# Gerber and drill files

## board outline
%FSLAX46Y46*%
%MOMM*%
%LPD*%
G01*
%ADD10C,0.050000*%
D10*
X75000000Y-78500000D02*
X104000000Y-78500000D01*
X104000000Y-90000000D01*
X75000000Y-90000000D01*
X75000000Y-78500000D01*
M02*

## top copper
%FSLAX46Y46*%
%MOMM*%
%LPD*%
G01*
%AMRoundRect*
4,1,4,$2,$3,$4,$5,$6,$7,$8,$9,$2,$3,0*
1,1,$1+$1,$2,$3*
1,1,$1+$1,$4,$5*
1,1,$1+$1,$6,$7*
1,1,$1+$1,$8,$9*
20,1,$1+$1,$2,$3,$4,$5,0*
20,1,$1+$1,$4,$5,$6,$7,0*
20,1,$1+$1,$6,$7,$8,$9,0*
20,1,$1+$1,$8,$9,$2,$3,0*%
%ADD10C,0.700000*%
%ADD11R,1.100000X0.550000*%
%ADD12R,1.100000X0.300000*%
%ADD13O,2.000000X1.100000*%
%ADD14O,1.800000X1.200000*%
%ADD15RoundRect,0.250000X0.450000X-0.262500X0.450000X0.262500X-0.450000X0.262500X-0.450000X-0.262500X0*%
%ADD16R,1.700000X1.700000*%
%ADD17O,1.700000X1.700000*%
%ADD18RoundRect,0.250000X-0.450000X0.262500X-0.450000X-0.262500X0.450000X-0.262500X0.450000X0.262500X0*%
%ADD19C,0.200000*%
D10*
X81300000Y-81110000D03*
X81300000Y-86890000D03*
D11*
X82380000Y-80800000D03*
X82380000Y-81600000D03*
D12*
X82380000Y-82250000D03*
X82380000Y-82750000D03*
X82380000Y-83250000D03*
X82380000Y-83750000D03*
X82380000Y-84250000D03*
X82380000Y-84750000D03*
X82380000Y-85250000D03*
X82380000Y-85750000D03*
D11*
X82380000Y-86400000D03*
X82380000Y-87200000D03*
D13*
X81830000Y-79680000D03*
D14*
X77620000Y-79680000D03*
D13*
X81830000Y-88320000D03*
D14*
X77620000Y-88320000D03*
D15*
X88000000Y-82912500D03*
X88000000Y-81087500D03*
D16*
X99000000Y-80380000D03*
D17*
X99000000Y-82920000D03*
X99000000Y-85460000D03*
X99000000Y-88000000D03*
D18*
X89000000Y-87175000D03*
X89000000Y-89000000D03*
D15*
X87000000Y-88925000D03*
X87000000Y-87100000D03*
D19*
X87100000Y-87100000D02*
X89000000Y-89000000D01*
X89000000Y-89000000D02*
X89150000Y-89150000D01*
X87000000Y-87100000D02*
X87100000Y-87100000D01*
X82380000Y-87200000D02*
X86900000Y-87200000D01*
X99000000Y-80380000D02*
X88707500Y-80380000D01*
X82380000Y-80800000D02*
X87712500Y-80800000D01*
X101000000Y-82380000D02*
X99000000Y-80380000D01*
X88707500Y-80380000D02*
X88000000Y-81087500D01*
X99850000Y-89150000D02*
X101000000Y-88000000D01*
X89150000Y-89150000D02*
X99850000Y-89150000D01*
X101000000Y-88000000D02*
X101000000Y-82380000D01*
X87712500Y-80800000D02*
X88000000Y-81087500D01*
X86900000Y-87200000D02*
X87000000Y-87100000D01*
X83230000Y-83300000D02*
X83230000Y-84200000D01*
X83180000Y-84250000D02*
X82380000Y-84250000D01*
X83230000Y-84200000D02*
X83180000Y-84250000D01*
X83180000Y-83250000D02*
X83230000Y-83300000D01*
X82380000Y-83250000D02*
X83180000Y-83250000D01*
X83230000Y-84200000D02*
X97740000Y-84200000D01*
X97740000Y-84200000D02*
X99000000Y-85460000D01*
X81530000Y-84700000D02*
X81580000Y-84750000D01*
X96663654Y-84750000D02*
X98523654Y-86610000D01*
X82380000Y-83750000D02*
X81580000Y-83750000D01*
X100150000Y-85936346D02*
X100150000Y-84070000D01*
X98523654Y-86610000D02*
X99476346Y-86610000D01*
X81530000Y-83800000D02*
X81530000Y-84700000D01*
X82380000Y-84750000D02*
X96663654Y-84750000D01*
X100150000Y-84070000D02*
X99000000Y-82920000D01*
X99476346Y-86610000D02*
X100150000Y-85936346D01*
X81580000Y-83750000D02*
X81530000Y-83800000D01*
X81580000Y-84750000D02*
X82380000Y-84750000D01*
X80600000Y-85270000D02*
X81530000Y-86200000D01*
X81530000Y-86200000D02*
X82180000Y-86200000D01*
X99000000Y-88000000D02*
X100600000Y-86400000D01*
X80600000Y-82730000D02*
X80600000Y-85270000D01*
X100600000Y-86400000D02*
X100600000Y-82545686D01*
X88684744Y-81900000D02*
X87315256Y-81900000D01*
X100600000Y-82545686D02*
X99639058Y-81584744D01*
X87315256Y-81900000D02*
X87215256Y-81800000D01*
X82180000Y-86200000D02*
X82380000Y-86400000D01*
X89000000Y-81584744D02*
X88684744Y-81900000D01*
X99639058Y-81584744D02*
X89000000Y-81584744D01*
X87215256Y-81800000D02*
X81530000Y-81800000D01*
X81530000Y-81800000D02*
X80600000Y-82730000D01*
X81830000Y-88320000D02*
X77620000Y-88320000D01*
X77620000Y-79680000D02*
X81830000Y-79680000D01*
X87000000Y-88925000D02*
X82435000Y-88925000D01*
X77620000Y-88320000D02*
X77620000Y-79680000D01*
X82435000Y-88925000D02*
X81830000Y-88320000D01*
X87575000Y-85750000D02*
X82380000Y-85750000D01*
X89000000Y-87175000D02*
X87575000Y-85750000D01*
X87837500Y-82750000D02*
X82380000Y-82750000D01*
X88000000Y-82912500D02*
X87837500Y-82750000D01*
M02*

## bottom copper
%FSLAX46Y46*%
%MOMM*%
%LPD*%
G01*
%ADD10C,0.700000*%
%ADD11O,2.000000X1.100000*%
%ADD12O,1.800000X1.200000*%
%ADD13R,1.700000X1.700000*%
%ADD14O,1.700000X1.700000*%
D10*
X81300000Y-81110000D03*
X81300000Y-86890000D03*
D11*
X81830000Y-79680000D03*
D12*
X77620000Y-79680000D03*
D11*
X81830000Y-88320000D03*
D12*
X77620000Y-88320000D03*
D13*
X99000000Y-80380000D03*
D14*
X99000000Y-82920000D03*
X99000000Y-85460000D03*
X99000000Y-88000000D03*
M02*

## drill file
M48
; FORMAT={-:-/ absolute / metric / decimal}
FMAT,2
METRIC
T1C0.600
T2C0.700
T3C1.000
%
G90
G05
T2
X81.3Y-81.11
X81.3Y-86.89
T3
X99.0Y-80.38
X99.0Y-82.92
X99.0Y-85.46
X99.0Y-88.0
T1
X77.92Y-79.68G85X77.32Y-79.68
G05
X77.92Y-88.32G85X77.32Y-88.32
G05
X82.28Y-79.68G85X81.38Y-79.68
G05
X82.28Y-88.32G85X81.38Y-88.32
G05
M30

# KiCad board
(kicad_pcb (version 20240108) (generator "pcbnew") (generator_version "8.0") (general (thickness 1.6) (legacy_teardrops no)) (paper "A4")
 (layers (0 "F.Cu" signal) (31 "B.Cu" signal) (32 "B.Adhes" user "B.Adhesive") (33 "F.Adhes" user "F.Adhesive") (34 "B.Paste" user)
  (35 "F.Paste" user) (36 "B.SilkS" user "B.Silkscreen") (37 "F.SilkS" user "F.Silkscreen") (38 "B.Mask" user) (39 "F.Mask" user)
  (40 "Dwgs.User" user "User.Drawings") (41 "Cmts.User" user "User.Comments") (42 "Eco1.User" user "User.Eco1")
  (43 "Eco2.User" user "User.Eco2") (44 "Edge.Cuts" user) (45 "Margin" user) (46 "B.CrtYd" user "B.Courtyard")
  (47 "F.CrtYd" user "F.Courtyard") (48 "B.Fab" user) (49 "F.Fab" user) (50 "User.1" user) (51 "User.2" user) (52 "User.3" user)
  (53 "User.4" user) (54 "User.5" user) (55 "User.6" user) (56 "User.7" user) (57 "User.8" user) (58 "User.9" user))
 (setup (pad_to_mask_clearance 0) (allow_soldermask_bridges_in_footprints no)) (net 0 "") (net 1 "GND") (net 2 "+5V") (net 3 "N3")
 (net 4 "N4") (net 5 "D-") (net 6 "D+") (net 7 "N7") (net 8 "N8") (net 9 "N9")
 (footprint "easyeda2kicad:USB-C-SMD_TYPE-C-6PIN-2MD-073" (layer "F.Cu") (at 80 84 -90)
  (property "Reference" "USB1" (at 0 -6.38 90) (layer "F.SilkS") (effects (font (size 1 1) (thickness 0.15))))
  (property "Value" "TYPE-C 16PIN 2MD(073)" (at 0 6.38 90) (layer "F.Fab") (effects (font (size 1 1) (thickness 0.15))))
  (pad "" thru_hole circle (at -2.89 -1.3 270) (size 0.7 0.7) (drill 0.7) (layers "*.Cu" "*.Mask") (remove_unused_layers no))
  (pad "" thru_hole circle (at 2.89 -1.3 270) (size 0.7 0.7) (drill 0.7) (layers "*.Cu" "*.Mask") (remove_unused_layers no))
  (pad "1" smd rect (at -3.2 -2.38 270) (size 0.55 1.1) (layers "F.Cu" "F.Paste" "F.Mask") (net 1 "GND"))
  (pad "2" smd rect (at -2.4 -2.38 270) (size 0.55 1.1) (layers "F.Cu" "F.Paste" "F.Mask") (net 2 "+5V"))
  (pad "3" smd rect (at -1.75 -2.38 270) (size 0.3 1.1) (layers "F.Cu" "F.Paste" "F.Mask") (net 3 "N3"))
  (pad "4" smd rect (at -1.25 -2.38 270) (size 0.3 1.1) (layers "F.Cu" "F.Paste" "F.Mask") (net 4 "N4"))
  (pad "5" smd rect (at -0.75 -2.38 270) (size 0.3 1.1) (layers "F.Cu" "F.Paste" "F.Mask") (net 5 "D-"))
  (pad "6" smd rect (at -0.25 -2.38 270) (size 0.3 1.1) (layers "F.Cu" "F.Paste" "F.Mask") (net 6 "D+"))
  (pad "7" smd rect (at 0.25 -2.38 270) (size 0.3 1.1) (layers "F.Cu" "F.Paste" "F.Mask") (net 5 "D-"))
  (pad "8" smd rect (at 0.75 -2.38 270) (size 0.3 1.1) (layers "F.Cu" "F.Paste" "F.Mask") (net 6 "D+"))
  (pad "9" smd rect (at 1.25 -2.38 270) (size 0.3 1.1) (layers "F.Cu" "F.Paste" "F.Mask") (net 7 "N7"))
  (pad "10" smd rect (at 1.75 -2.38 270) (size 0.3 1.1) (layers "F.Cu" "F.Paste" "F.Mask") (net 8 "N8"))
  (pad "11" smd rect (at 2.4 -2.38 270) (size 0.55 1.1) (layers "F.Cu" "F.Paste" "F.Mask") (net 2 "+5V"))
  (pad "12" smd rect (at 3.2 -2.38 270) (size 0.55 1.1) (layers "F.Cu" "F.Paste" "F.Mask") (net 1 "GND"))
  (pad "13" thru_hole oval (at -4.32 -1.83 270) (size 1.1 2) (drill oval 0.599999 1.499997) (layers "*.Cu" "*.Mask")
   (remove_unused_layers no) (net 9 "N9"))
  (pad "13" thru_hole oval (at -4.32 2.38 270) (size 1.2 1.8) (drill oval 0.599999 1.199998) (layers "*.Cu" "*.Mask")
   (remove_unused_layers no) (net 9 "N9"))
  (pad "14" thru_hole oval (at 4.32 -1.83 270) (size 1.1 2) (drill oval 0.599999 1.500022) (layers "*.Cu" "*.Mask")
   (remove_unused_layers no) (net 9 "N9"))
  (pad "14" thru_hole oval (at 4.32 2.38 270) (size 1.2 1.8) (drill oval 0.599999 1.199998) (layers "*.Cu" "*.Mask")
   (remove_unused_layers no) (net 9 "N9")))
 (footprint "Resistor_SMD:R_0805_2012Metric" (layer "F.Cu") (at 88 82 90)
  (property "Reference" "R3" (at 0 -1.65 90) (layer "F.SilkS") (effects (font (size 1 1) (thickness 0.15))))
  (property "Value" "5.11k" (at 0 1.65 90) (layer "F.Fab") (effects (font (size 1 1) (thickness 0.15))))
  (pad "1" smd roundrect (at -0.9125 0 90) (size 1.025 1.4) (layers "F.Cu" "F.Paste" "F.Mask") (roundrect_rratio 0.243902) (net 4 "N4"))
  (pad "2" smd roundrect (at 0.9125 0 90) (size 1.025 1.4) (layers "F.Cu" "F.Paste" "F.Mask") (roundrect_rratio 0.243902) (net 1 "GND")))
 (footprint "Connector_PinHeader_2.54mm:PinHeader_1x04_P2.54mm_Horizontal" (layer "F.Cu") (at 99 80.38)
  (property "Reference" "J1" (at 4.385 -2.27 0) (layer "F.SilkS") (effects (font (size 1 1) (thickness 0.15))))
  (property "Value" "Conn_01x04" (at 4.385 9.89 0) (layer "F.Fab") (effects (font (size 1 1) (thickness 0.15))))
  (pad "1" thru_hole rect (at 0 0) (size 1.7 1.7) (drill 1) (layers "*.Cu" "*.Mask") (remove_unused_layers no) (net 1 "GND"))
  (pad "2" thru_hole oval (at 0 2.54) (size 1.7 1.7) (drill 1) (layers "*.Cu" "*.Mask") (remove_unused_layers no) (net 6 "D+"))
  (pad "3" thru_hole oval (at 0 5.08) (size 1.7 1.7) (drill 1) (layers "*.Cu" "*.Mask") (remove_unused_layers no) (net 5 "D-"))
  (pad "4" thru_hole oval (at 0 7.62) (size 1.7 1.7) (drill 1) (layers "*.Cu" "*.Mask") (remove_unused_layers no) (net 2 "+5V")))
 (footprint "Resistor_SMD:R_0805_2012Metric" (layer "F.Cu") (at 89 88.0875 -90)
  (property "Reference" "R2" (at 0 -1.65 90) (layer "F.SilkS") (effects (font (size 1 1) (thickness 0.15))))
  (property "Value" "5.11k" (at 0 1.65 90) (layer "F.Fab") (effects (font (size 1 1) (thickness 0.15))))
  (pad "1" smd roundrect (at -0.9125 0 270) (size 1.025 1.4) (layers "F.Cu" "F.Paste" "F.Mask") (roundrect_rratio 0.243902) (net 8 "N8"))
  (pad "2" smd roundrect (at 0.9125 0 270) (size 1.025 1.4) (layers "F.Cu" "F.Paste" "F.Mask") (roundrect_rratio 0.243902) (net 1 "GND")))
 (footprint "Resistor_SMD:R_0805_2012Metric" (layer "F.Cu") (at 87 88.0125 90)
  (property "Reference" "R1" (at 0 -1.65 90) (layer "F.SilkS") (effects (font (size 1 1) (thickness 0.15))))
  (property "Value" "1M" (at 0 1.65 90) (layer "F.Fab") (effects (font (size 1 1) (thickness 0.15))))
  (pad "1" smd roundrect (at -0.9125 0 90) (size 1.025 1.4) (layers "F.Cu" "F.Paste" "F.Mask") (roundrect_rratio 0.243902) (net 9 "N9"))
  (pad "2" smd roundrect (at 0.9125 0 90) (size 1.025 1.4) (layers "F.Cu" "F.Paste" "F.Mask") (roundrect_rratio 0.243902) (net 1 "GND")))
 (gr_rect (start 75 78.5) (end 104 90) (stroke (width 0.05) (type default)) (fill none) (layer "Edge.Cuts"))
 (segment (start 87.1 87.1) (end 89 89) (width 0.2) (layer "F.Cu") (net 1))
 (segment (start 89 89) (end 89.15 89.15) (width 0.2) (layer "F.Cu") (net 1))
 (segment (start 87 87.1) (end 87.1 87.1) (width 0.2) (layer "F.Cu") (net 1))
 (segment (start 82.38 87.2) (end 86.9 87.2) (width 0.2) (layer "F.Cu") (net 1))
 (segment (start 99 80.38) (end 88.7075 80.38) (width 0.2) (layer "F.Cu") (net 1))
 (segment (start 82.38 80.8) (end 87.7125 80.8) (width 0.2) (layer "F.Cu") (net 1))
 (segment (start 101 82.38) (end 99 80.38) (width 0.2) (layer "F.Cu") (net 1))
 (segment (start 88.7075 80.38) (end 88 81.0875) (width 0.2) (layer "F.Cu") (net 1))
 (segment (start 99.85 89.15) (end 101 88) (width 0.2) (layer "F.Cu") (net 1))
 (segment (start 89.15 89.15) (end 99.85 89.15) (width 0.2) (layer "F.Cu") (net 1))
 (segment (start 101 88) (end 101 82.38) (width 0.2) (layer "F.Cu") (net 1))
 (segment (start 87.7125 80.8) (end 88 81.0875) (width 0.2) (layer "F.Cu") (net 1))
 (segment (start 86.9 87.2) (end 87 87.1) (width 0.2) (layer "F.Cu") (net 1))
 (segment (start 83.23 83.3) (end 83.23 84.2) (width 0.2) (layer "F.Cu") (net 5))
 (segment (start 83.18 84.25) (end 82.38 84.25) (width 0.2) (layer "F.Cu") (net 5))
 (segment (start 83.23 84.2) (end 83.18 84.25) (width 0.2) (layer "F.Cu") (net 5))
 (segment (start 83.18 83.25) (end 83.23 83.3) (width 0.2) (layer "F.Cu") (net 5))
 (segment (start 82.38 83.25) (end 83.18 83.25) (width 0.2) (layer "F.Cu") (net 5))
 (segment (start 83.23 84.2) (end 97.74 84.2) (width 0.2) (layer "F.Cu") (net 5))
 (segment (start 97.74 84.2) (end 99 85.46) (width 0.2) (layer "F.Cu") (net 5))
 (segment (start 81.53 84.7) (end 81.58 84.75) (width 0.2) (layer "F.Cu") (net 6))
 (segment (start 96.663654 84.75) (end 98.523654 86.61) (width 0.2) (layer "F.Cu") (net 6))
 (segment (start 82.38 83.75) (end 81.58 83.75) (width 0.2) (layer "F.Cu") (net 6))
 (segment (start 100.15 85.936346) (end 100.15 84.07) (width 0.2) (layer "F.Cu") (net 6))
 (segment (start 98.523654 86.61) (end 99.476346 86.61) (width 0.2) (layer "F.Cu") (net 6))
 (segment (start 81.53 83.8) (end 81.53 84.7) (width 0.2) (layer "F.Cu") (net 6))
 (segment (start 82.38 84.75) (end 96.663654 84.75) (width 0.2) (layer "F.Cu") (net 6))
 (segment (start 100.15 84.07) (end 99 82.92) (width 0.2) (layer "F.Cu") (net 6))
 (segment (start 99.476346 86.61) (end 100.15 85.936346) (width 0.2) (layer "F.Cu") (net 6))
 (segment (start 81.58 83.75) (end 81.53 83.8) (width 0.2) (layer "F.Cu") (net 6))
 (segment (start 81.58 84.75) (end 82.38 84.75) (width 0.2) (layer "F.Cu") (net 6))
 (segment (start 80.6 85.27) (end 81.53 86.2) (width 0.2) (layer "F.Cu") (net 2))
 (segment (start 81.53 86.2) (end 82.18 86.2) (width 0.2) (layer "F.Cu") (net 2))
 (segment (start 99 88) (end 100.6 86.4) (width 0.2) (layer "F.Cu") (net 2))
 (segment (start 80.6 82.73) (end 80.6 85.27) (width 0.2) (layer "F.Cu") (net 2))
 (segment (start 100.6 86.4) (end 100.6 82.545686) (width 0.2) (layer "F.Cu") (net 2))
 (segment (start 88.684744 81.9) (end 87.315256 81.9) (width 0.2) (layer "F.Cu") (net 2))
 (segment (start 100.6 82.545686) (end 99.639058 81.584744) (width 0.2) (layer "F.Cu") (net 2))
 (segment (start 87.315256 81.9) (end 87.215256 81.8) (width 0.2) (layer "F.Cu") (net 2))
 (segment (start 82.18 86.2) (end 82.38 86.4) (width 0.2) (layer "F.Cu") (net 2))
 (segment (start 89 81.584744) (end 88.684744 81.9) (width 0.2) (layer "F.Cu") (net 2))
 (segment (start 99.639058 81.584744) (end 89 81.584744) (width 0.2) (layer "F.Cu") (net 2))
 (segment (start 87.215256 81.8) (end 81.53 81.8) (width 0.2) (layer "F.Cu") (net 2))
 (segment (start 81.53 81.8) (end 80.6 82.73) (width 0.2) (layer "F.Cu") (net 2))
 (segment (start 81.83 88.32) (end 77.62 88.32) (width 0.2) (layer "F.Cu") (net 9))
 (segment (start 77.62 79.68) (end 81.83 79.68) (width 0.2) (layer "F.Cu") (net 9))
 (segment (start 87 88.925) (end 82.435 88.925) (width 0.2) (layer "F.Cu") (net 9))
 (segment (start 77.62 88.32) (end 77.62 79.68) (width 0.2) (layer "F.Cu") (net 9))
 (segment (start 82.435 88.925) (end 81.83 88.32) (width 0.2) (layer "F.Cu") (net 9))
 (segment (start 87.575 85.75) (end 82.38 85.75) (width 0.2) (layer "F.Cu") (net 8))
 (segment (start 89 87.175) (end 87.575 85.75) (width 0.2) (layer "F.Cu") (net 8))
 (segment (start 87.8375 82.75) (end 82.38 82.75) (width 0.2) (layer "F.Cu") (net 4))
 (segment (start 88 82.9125) (end 87.8375 82.75) (width 0.2) (layer "F.Cu") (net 4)))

